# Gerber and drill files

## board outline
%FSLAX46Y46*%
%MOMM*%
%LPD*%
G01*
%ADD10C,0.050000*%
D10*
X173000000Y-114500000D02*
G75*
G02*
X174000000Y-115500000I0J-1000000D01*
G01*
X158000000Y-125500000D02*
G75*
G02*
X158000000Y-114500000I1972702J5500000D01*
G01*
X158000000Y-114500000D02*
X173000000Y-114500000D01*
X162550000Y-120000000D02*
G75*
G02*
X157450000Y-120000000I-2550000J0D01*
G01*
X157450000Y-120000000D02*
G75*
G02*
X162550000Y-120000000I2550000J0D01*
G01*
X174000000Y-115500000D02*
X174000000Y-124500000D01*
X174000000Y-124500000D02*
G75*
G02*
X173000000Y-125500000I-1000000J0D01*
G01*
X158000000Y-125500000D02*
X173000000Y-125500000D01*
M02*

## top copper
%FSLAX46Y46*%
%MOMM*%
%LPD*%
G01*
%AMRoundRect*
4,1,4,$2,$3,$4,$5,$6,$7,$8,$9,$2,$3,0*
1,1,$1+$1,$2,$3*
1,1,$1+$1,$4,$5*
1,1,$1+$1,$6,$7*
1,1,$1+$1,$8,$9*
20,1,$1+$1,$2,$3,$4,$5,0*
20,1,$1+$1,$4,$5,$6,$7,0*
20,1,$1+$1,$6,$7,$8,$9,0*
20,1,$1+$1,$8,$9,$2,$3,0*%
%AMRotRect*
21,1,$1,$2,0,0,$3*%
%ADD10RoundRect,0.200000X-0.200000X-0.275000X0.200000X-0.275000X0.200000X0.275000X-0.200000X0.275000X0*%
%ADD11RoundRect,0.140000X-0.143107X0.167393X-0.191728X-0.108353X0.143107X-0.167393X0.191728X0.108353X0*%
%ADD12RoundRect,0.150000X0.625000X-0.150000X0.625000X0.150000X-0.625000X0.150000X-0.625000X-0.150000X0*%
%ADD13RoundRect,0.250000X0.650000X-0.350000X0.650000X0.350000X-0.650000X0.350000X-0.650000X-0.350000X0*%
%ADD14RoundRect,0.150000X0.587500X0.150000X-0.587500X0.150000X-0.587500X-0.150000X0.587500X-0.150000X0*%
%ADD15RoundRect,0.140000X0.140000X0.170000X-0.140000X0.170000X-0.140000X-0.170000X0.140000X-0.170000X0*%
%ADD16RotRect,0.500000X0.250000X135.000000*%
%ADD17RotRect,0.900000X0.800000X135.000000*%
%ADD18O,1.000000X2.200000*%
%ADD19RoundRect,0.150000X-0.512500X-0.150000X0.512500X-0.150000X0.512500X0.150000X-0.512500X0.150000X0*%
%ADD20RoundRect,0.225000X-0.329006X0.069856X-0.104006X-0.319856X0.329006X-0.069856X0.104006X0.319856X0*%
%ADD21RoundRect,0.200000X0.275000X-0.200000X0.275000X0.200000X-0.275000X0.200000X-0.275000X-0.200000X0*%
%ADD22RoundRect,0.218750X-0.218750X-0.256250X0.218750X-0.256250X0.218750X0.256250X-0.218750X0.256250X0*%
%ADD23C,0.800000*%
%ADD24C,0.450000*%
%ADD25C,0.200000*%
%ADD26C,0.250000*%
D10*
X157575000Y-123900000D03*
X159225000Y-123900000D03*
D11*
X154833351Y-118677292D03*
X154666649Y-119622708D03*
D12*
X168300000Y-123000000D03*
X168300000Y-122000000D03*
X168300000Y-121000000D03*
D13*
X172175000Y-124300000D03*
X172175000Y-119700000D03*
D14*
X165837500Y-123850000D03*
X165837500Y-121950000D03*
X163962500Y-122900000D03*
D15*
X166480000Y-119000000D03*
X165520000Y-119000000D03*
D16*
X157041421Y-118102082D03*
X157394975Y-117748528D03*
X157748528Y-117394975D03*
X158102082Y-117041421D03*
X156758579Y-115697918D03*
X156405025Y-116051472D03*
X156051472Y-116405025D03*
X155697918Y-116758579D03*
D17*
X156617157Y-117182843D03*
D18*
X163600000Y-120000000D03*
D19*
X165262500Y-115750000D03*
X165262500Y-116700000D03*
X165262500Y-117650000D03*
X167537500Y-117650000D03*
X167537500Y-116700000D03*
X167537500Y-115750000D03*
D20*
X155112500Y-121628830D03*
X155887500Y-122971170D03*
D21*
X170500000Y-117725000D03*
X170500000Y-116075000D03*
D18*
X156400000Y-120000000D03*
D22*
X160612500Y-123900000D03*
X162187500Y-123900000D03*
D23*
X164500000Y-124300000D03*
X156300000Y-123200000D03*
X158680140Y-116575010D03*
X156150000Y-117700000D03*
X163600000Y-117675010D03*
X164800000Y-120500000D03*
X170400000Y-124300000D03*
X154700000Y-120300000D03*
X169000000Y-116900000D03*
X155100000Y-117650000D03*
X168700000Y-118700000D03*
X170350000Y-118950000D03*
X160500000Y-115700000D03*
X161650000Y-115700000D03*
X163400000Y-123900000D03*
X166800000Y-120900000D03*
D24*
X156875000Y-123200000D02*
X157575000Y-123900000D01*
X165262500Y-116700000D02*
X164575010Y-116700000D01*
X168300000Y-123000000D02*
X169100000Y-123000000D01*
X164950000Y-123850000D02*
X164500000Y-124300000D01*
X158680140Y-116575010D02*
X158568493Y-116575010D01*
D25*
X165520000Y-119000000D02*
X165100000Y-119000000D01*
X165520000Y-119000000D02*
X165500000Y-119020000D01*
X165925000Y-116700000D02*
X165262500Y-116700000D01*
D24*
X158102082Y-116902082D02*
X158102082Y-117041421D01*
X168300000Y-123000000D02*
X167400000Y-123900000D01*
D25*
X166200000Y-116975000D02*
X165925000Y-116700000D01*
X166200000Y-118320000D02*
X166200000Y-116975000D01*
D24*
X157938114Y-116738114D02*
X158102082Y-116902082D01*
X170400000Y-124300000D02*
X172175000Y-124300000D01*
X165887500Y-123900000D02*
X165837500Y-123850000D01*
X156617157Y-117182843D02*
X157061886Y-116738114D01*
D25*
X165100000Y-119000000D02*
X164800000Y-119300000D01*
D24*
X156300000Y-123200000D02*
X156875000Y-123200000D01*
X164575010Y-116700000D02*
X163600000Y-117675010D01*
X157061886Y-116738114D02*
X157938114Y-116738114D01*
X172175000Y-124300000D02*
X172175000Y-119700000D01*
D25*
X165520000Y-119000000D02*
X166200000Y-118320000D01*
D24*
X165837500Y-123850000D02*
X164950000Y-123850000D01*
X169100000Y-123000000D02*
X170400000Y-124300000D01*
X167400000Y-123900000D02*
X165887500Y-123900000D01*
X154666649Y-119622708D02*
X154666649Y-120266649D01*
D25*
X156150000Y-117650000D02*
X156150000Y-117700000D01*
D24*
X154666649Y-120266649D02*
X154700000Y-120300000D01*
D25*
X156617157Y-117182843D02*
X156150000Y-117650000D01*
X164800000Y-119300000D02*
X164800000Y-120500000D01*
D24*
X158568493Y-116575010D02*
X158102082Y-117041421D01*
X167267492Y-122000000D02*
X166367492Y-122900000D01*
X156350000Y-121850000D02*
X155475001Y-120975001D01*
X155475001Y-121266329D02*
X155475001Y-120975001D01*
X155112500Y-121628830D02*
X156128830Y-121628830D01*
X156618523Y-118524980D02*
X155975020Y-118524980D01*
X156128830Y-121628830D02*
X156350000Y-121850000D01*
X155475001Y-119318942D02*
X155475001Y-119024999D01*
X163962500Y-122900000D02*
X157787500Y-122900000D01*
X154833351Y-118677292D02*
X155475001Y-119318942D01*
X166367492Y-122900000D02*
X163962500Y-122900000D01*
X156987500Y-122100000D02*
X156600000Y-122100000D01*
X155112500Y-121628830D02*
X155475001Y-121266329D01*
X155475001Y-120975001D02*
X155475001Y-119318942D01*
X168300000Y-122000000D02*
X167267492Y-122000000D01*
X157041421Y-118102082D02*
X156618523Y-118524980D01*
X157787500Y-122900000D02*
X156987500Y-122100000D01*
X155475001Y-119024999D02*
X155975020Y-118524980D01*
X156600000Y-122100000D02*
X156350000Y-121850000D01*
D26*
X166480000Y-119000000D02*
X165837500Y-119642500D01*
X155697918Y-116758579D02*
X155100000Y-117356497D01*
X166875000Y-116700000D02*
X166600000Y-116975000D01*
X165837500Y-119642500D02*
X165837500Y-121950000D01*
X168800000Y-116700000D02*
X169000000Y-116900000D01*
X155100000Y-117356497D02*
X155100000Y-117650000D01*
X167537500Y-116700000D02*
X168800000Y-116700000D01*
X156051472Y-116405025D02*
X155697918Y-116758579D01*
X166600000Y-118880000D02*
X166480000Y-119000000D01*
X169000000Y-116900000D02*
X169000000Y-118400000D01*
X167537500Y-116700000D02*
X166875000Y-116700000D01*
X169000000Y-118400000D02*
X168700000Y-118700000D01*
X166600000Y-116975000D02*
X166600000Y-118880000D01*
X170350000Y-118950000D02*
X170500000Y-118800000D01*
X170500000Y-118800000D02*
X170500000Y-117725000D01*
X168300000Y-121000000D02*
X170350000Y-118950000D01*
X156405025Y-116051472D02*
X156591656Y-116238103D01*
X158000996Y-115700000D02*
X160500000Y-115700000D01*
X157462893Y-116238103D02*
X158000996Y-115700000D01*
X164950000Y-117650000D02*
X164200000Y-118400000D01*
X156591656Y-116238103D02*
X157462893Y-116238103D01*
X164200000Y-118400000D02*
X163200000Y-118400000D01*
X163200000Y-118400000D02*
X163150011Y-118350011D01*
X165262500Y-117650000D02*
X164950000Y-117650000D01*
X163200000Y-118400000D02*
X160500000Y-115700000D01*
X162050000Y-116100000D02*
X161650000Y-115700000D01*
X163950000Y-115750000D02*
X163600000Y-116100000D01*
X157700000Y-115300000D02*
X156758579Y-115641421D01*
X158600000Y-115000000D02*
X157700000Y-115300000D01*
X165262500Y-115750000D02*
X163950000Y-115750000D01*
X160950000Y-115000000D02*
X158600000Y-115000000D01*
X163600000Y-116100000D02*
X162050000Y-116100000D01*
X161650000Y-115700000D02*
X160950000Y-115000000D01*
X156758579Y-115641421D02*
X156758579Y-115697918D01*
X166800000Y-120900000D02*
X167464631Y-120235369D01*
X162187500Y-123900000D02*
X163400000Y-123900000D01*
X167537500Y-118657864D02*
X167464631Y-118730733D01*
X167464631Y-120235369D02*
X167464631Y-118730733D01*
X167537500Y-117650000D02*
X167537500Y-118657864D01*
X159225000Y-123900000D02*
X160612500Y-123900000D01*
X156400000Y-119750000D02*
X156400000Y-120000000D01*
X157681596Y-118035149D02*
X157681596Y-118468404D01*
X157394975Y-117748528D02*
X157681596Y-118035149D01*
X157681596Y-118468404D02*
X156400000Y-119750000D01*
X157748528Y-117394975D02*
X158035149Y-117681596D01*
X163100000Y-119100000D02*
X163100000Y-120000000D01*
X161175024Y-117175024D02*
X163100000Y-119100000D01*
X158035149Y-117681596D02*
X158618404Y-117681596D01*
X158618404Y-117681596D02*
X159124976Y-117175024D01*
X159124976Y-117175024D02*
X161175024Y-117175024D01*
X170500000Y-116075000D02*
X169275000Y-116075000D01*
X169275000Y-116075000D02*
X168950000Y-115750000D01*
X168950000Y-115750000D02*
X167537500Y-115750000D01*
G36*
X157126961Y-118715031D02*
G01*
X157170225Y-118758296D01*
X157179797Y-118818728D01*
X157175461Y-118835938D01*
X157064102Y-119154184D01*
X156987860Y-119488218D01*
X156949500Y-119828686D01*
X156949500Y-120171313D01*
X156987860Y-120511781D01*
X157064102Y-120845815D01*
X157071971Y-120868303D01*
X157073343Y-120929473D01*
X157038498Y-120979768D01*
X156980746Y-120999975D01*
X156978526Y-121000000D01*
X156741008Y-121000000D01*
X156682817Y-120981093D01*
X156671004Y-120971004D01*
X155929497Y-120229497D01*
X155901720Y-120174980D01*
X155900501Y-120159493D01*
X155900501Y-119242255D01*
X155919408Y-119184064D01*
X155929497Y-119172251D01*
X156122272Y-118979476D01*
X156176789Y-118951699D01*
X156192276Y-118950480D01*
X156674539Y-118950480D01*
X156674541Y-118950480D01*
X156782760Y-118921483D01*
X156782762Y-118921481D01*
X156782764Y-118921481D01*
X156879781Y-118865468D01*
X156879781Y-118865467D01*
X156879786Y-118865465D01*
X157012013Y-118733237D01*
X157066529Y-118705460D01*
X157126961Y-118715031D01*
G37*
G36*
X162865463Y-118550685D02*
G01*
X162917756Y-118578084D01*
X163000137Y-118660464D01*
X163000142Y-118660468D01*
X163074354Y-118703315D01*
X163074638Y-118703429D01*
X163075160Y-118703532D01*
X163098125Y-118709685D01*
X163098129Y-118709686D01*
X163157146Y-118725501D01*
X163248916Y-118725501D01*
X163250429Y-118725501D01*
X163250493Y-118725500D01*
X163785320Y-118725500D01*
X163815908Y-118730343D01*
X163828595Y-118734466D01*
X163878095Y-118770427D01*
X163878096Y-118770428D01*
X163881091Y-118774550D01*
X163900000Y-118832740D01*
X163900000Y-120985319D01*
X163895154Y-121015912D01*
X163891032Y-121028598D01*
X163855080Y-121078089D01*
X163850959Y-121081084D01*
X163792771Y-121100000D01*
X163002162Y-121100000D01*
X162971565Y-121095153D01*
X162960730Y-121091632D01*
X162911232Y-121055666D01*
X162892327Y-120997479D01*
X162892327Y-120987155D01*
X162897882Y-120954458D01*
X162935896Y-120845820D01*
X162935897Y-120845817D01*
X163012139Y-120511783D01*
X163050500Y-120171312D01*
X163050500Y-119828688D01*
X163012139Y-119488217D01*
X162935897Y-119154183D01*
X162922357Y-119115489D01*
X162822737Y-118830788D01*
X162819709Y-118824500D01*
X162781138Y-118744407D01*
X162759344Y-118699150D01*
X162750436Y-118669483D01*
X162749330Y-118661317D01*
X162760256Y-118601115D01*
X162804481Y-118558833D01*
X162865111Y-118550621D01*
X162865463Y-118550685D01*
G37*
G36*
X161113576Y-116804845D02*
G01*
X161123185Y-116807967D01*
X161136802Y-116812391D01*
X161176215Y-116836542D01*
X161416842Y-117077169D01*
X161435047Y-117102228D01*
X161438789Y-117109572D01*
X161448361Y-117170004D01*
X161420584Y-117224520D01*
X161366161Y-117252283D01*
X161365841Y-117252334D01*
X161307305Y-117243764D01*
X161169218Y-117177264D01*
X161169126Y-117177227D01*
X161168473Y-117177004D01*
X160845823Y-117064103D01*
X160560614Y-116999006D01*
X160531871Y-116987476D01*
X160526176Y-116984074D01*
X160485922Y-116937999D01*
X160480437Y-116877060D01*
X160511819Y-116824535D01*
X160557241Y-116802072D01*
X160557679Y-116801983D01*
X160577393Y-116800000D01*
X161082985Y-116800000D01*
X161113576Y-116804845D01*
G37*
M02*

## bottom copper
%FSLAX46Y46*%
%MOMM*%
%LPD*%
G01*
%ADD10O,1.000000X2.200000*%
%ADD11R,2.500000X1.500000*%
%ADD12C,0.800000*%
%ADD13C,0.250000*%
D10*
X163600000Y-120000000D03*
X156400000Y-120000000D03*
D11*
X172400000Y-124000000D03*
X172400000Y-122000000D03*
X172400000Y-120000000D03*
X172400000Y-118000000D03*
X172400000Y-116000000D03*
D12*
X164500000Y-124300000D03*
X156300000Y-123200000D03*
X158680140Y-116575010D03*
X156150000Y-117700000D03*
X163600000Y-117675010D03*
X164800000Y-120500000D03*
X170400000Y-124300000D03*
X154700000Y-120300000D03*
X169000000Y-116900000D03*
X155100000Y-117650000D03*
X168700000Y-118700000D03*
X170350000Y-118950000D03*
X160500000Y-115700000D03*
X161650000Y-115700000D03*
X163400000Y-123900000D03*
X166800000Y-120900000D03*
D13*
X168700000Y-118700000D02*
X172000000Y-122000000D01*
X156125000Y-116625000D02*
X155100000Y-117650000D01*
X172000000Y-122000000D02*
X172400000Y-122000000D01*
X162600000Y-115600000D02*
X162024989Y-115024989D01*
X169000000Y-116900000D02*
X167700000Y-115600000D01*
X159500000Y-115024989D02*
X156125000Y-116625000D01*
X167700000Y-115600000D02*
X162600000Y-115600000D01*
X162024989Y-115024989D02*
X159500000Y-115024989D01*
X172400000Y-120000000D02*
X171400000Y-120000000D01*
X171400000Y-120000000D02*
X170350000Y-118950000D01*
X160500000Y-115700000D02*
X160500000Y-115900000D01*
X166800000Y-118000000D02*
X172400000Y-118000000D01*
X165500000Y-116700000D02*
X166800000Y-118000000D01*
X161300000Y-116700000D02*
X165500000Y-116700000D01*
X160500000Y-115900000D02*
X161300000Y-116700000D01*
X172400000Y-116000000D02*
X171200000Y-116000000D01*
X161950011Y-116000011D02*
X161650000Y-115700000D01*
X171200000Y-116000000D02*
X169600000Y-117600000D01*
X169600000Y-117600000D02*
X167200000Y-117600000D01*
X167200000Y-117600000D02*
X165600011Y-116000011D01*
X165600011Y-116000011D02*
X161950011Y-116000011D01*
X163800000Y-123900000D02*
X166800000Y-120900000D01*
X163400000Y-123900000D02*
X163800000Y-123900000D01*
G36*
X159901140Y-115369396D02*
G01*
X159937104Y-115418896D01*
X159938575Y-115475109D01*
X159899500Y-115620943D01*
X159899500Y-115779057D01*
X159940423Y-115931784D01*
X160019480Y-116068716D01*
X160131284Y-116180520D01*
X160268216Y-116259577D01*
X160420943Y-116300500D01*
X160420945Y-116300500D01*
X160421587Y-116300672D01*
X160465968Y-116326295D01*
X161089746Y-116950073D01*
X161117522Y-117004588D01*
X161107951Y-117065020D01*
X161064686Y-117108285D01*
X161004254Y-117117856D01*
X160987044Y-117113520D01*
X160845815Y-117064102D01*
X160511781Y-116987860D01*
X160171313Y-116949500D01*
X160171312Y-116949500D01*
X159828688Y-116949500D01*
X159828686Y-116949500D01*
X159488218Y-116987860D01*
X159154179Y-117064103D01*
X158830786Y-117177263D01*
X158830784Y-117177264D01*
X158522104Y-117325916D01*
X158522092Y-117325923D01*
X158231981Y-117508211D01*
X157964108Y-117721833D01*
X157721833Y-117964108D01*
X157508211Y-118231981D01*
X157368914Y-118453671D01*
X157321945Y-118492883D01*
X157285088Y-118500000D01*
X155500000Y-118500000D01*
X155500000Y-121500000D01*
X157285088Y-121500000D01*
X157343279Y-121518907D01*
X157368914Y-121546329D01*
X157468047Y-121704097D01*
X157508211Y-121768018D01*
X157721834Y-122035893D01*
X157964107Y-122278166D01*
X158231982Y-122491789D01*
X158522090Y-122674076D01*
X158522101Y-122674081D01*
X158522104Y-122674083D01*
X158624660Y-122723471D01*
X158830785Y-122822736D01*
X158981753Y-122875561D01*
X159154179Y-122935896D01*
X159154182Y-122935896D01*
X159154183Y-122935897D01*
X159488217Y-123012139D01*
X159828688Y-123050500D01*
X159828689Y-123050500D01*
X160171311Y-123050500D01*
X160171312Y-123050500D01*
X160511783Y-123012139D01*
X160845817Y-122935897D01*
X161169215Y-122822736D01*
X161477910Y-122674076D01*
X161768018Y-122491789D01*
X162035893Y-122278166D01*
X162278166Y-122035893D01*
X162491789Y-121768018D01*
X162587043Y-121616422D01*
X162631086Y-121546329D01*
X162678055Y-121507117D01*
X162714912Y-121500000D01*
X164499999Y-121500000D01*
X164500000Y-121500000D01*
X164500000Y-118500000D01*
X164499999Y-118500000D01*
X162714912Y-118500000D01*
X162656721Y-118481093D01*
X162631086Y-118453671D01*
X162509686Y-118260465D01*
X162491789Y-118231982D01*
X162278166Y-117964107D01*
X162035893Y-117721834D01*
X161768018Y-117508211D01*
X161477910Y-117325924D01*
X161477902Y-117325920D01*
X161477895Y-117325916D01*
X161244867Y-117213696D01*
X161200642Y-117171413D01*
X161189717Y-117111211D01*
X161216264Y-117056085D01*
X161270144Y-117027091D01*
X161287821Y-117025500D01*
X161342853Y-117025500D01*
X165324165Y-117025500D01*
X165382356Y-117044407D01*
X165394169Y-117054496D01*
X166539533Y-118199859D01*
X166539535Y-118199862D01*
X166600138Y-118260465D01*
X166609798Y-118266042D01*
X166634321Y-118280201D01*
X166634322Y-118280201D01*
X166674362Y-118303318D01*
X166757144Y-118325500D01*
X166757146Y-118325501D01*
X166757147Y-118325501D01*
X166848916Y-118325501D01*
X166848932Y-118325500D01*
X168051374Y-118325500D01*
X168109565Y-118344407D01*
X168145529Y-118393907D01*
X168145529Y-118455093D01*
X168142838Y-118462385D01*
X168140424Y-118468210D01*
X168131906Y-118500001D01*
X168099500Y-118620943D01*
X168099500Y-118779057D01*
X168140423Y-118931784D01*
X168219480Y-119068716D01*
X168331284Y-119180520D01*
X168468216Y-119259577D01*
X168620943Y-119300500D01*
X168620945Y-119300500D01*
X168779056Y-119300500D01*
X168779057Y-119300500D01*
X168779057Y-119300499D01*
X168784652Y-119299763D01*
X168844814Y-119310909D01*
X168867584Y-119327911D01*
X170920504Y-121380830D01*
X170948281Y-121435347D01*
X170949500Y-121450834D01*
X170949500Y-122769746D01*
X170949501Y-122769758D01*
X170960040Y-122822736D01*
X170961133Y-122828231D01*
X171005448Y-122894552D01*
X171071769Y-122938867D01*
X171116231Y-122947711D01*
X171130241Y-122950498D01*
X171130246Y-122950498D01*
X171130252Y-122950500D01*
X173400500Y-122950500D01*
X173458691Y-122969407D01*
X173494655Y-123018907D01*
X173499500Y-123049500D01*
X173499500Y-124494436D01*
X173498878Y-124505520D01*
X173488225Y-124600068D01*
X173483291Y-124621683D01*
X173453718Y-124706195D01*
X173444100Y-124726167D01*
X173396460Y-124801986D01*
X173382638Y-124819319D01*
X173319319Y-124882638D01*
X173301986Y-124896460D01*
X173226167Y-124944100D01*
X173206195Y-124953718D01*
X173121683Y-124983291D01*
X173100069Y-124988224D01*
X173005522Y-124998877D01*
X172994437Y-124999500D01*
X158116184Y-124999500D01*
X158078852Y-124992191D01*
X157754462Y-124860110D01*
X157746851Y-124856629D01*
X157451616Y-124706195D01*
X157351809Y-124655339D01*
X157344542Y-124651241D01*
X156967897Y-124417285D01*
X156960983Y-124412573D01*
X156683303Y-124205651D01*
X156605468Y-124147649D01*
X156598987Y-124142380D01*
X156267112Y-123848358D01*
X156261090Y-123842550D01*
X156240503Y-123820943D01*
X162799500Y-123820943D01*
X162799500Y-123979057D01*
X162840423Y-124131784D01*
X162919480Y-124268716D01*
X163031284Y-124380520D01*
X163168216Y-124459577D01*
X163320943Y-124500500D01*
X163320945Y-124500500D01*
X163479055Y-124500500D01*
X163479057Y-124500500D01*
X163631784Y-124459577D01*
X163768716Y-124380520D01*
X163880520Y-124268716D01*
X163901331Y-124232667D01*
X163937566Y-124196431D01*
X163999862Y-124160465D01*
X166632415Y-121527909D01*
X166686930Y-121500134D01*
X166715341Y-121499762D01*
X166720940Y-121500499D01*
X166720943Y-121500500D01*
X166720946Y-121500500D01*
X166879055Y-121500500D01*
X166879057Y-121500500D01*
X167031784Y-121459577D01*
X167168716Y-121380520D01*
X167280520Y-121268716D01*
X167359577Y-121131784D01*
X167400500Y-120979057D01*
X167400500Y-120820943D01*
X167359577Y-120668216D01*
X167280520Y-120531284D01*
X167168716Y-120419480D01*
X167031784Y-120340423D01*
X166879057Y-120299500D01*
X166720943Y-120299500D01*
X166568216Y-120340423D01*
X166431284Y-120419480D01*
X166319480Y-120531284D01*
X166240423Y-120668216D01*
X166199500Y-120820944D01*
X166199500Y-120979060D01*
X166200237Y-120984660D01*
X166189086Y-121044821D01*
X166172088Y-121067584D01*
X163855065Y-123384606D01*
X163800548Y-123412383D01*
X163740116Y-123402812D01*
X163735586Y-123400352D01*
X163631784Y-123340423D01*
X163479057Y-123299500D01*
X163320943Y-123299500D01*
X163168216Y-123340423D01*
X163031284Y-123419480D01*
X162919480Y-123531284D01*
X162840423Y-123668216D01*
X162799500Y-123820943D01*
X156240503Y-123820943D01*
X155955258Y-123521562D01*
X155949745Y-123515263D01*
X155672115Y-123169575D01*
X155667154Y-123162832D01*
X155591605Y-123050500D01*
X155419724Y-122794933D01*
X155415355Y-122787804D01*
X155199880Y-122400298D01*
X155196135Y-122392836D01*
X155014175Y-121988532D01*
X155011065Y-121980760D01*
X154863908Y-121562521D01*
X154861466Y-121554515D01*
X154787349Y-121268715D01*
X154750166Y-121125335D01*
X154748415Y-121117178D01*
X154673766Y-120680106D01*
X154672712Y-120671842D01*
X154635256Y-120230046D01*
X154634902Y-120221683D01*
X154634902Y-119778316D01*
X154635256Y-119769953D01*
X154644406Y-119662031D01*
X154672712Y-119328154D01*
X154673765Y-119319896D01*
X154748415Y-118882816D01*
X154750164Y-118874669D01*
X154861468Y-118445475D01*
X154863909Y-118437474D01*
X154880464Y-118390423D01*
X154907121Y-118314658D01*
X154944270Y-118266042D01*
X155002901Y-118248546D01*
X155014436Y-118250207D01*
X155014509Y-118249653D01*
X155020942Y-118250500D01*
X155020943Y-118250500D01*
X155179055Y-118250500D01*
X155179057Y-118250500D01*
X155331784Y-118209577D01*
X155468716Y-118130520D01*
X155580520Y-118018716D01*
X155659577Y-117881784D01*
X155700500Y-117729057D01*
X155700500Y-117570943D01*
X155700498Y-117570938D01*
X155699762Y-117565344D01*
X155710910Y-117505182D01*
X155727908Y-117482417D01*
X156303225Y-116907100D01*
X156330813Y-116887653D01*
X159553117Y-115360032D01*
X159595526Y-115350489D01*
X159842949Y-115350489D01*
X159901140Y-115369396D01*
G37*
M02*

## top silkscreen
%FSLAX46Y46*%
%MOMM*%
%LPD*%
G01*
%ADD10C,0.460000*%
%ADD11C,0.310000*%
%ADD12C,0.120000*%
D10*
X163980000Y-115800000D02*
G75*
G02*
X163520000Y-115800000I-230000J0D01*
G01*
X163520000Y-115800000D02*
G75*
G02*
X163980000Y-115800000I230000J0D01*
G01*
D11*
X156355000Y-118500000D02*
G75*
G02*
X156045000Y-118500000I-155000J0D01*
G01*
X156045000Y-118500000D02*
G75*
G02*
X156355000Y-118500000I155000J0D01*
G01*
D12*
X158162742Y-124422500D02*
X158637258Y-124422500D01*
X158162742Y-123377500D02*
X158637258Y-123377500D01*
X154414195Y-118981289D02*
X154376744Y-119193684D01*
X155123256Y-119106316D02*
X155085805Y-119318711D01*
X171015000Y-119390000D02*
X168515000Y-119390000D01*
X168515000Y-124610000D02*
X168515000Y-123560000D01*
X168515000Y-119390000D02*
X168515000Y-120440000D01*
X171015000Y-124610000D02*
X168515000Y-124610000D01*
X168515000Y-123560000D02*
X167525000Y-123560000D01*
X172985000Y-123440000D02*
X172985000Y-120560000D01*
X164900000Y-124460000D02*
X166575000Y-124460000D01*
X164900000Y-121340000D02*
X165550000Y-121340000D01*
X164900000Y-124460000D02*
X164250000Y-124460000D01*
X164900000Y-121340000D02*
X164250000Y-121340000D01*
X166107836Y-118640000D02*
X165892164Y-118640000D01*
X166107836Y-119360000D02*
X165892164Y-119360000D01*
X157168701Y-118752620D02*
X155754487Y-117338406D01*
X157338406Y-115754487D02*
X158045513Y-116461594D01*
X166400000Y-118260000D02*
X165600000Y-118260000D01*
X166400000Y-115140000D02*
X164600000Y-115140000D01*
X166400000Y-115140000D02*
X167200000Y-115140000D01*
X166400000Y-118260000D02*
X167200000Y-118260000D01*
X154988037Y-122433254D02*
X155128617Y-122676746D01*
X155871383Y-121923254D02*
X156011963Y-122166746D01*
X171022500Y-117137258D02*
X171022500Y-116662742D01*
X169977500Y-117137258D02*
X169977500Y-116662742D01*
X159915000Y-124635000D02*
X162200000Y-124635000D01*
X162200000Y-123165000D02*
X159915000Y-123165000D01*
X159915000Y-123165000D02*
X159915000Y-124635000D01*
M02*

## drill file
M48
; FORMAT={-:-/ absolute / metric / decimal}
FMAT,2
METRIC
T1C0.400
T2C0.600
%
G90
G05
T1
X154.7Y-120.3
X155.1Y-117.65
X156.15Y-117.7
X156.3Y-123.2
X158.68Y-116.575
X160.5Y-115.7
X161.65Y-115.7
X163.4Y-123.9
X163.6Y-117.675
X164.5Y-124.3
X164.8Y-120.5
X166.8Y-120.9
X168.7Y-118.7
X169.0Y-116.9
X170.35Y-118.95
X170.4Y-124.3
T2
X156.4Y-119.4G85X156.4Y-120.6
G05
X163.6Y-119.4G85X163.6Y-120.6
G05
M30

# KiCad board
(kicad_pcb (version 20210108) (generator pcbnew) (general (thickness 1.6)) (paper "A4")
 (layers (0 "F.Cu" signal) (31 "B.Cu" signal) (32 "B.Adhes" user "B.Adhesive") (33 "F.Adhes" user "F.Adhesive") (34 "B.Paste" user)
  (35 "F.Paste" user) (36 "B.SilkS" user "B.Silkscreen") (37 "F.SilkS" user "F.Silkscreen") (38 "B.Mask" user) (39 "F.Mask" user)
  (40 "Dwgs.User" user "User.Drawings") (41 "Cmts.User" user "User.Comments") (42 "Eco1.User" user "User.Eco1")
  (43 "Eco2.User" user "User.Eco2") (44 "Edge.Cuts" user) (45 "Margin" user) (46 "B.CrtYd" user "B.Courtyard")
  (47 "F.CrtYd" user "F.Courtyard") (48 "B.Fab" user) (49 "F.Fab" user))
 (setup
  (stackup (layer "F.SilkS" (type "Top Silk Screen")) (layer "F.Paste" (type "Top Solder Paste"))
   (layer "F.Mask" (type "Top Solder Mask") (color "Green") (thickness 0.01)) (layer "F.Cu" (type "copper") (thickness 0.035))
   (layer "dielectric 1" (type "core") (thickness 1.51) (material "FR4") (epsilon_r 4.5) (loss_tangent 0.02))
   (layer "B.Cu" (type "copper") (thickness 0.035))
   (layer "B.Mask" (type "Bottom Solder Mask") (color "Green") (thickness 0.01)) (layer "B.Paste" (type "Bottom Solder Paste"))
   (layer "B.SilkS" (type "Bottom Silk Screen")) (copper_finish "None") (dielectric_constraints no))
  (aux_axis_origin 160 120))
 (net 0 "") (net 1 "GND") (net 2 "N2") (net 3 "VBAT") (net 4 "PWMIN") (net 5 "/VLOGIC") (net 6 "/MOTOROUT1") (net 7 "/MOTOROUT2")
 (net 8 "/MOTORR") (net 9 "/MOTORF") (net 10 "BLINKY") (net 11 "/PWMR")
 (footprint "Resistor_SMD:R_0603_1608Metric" (layer "F.Cu") (at 158.4 123.9)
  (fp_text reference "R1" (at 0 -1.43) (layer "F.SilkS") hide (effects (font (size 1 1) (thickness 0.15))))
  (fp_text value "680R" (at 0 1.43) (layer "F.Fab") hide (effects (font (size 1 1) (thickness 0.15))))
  (fp_line (start -0.237258 0.5225) (end 0.237258 0.5225) (layer "F.SilkS") (width 0.12))
  (fp_line (start -0.237258 -0.5225) (end 0.237258 -0.5225) (layer "F.SilkS") (width 0.12))
  (pad "1" smd roundrect (at -0.825 0) (locked) (size 0.8 0.95) (layers "F.Cu" "F.Paste" "F.Mask") (roundrect_rratio 0.25) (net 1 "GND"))
  (pad "2" smd roundrect (at 0.825 0) (locked) (size 0.8 0.95) (layers "F.Cu" "F.Paste" "F.Mask") (roundrect_rratio 0.25) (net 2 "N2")))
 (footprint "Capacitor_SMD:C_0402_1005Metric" (layer "F.Cu") (at 154.75 119.15 -100)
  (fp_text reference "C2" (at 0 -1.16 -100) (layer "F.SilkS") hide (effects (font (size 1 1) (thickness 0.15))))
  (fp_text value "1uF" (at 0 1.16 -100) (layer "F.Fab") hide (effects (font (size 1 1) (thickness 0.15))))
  (fp_line (start -0.107836 0.36) (end 0.107836 0.36) (layer "F.SilkS") (width 0.12))
  (fp_line (start -0.107836 -0.36) (end 0.107836 -0.36) (layer "F.SilkS") (width 0.12))
  (pad "1" smd roundrect (at -0.48 0 260) (locked) (size 0.56 0.62) (layers "F.Cu" "F.Paste" "F.Mask") (roundrect_rratio 0.25)
   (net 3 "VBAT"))
  (pad "2" smd roundrect (at 0.48 0 260) (locked) (size 0.56 0.62) (layers "F.Cu" "F.Paste" "F.Mask") (roundrect_rratio 0.25) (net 1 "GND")))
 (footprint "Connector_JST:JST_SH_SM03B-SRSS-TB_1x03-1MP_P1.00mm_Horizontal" (layer "F.Cu") (at 170.3 122 90)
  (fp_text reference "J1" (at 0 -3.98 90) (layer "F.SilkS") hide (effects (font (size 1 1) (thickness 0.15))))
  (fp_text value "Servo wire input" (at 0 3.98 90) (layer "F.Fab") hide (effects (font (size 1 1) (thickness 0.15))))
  (fp_line (start 2.61 0.715) (end 2.61 -1.785) (layer "F.SilkS") (width 0.12))
  (fp_line (start -2.61 -1.785) (end -1.56 -1.785) (layer "F.SilkS") (width 0.12))
  (fp_line (start 2.61 -1.785) (end 1.56 -1.785) (layer "F.SilkS") (width 0.12))
  (fp_line (start -2.61 0.715) (end -2.61 -1.785) (layer "F.SilkS") (width 0.12))
  (fp_line (start -1.56 -1.785) (end -1.56 -2.775) (layer "F.SilkS") (width 0.12))
  (fp_line (start -1.44 2.685) (end 1.44 2.685) (layer "F.SilkS") (width 0.12))
  (pad "1" smd roundrect (at -1 -2 90) (locked) (size 0.6 1.55) (layers "F.Cu" "F.Paste" "F.Mask") (roundrect_rratio 0.25) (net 1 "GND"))
  (pad "2" smd roundrect (at 0 -2 90) (locked) (size 0.6 1.55) (layers "F.Cu" "F.Paste" "F.Mask") (roundrect_rratio 0.25) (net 3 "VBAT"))
  (pad "3" smd roundrect (at 1 -2 90) (locked) (size 0.6 1.55) (layers "F.Cu" "F.Paste" "F.Mask") (roundrect_rratio 0.25) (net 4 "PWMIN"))
  (pad "MP" smd roundrect (at -2.3 1.875 90) (locked) (size 1.2 1.8) (layers "F.Cu" "F.Paste" "F.Mask") (roundrect_rratio 0.208333)
   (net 1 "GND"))
  (pad "MP" smd roundrect (at 2.3 1.875 90) (locked) (size 1.2 1.8) (layers "F.Cu" "F.Paste" "F.Mask") (roundrect_rratio 0.208333)
   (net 1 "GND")))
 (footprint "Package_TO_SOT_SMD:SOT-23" (layer "F.Cu") (at 164.9 122.9 180)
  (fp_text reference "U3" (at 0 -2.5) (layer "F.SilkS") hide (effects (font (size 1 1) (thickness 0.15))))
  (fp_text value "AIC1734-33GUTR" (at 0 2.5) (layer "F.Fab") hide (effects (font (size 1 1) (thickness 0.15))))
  (fp_line (start 0 -1.56) (end -1.675 -1.56) (layer "F.SilkS") (width 0.12))
  (fp_line (start 0 1.56) (end -0.65 1.56) (layer "F.SilkS") (width 0.12))
  (fp_line (start 0 -1.56) (end 0.65 -1.56) (layer "F.SilkS") (width 0.12))
  (fp_line (start 0 1.56) (end 0.65 1.56) (layer "F.SilkS") (width 0.12))
  (pad "1" smd roundrect (at -0.9375 -0.95 180) (locked) (size 1.475 0.6) (layers "F.Cu" "F.Paste" "F.Mask") (roundrect_rratio 0.25)
   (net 1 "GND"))
  (pad "2" smd roundrect (at -0.9375 0.95 180) (locked) (size 1.475 0.6) (layers "F.Cu" "F.Paste" "F.Mask") (roundrect_rratio 0.25)
   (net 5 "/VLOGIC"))
  (pad "3" smd roundrect (at 0.9375 0 180) (locked) (size 1.475 0.6) (layers "F.Cu" "F.Paste" "F.Mask") (roundrect_rratio 0.25)
   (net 3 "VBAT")))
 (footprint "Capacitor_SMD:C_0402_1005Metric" (layer "F.Cu") (at 166 119 180)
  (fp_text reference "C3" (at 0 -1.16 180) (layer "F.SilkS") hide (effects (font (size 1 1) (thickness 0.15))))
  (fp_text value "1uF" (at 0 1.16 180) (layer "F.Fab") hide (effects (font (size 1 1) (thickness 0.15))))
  (fp_line (start -0.107836 0.36) (end 0.107836 0.36) (layer "F.SilkS") (width 0.12))
  (fp_line (start -0.107836 -0.36) (end 0.107836 -0.36) (layer "F.SilkS") (width 0.12))
  (pad "1" smd roundrect (at -0.48 0 180) (locked) (size 0.56 0.62) (layers "F.Cu" "F.Paste" "F.Mask") (roundrect_rratio 0.25)
   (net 5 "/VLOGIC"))
  (pad "2" smd roundrect (at 0.48 0 180) (locked) (size 0.56 0.62) (layers "F.Cu" "F.Paste" "F.Mask") (roundrect_rratio 0.25) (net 1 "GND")))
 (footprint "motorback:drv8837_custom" (layer "F.Cu") (at 156.9 116.9 135)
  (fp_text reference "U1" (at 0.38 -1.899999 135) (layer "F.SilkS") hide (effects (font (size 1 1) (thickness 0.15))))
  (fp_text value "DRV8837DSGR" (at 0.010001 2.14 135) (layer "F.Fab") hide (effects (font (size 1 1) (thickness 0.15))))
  (fp_line (start -1.5 -1.12) (end 0.5 -1.12) (layer "F.SilkS") (width 0.12))
  (fp_line (start 0.5 1.12) (end -0.5 1.12) (layer "F.SilkS") (width 0.12))
  (pad "" smd rect (at 0 -0.4 135) (locked) (size 0.75 0.65) (layers "F.Paste"))
  (pad "1" smd rect (at -0.95 -0.75 135) (locked) (size 0.5 0.25) (layers "F.Cu" "F.Paste" "F.Mask") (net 3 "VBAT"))
  (pad "2" smd rect (at -0.95 -0.25 135) (locked) (size 0.5 0.25) (layers "F.Cu" "F.Paste" "F.Mask") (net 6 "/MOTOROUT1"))
  (pad "3" smd rect (at -0.95 0.25 135) (locked) (size 0.5 0.25) (layers "F.Cu" "F.Paste" "F.Mask") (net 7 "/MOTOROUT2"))
  (pad "4" smd rect (at -0.95 0.75 135) (locked) (size 0.5 0.25) (layers "F.Cu" "F.Paste" "F.Mask") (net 1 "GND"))
  (pad "5" smd rect (at 0.95 0.75 135) (locked) (size 0.5 0.25) (layers "F.Cu" "F.Paste" "F.Mask") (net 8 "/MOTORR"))
  (pad "6" smd rect (at 0.95 0.25 135) (locked) (size 0.5 0.25) (layers "F.Cu" "F.Paste" "F.Mask") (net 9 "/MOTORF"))
  (pad "7" smd rect (at 0.95 -0.25 135) (locked) (size 0.5 0.25) (layers "F.Cu" "F.Paste" "F.Mask") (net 5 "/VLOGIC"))
  (pad "8" smd rect (at 0.95 -0.75 135) (locked) (size 0.5 0.25) (layers "F.Cu" "F.Paste" "F.Mask") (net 5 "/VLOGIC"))
  (pad "9" smd rect (at 0 -0.4 135) (locked) (size 0.9 0.8) (layers "F.Cu" "F.Mask") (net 1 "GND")))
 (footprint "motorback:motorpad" (layer "F.Cu") (at 163.6 120)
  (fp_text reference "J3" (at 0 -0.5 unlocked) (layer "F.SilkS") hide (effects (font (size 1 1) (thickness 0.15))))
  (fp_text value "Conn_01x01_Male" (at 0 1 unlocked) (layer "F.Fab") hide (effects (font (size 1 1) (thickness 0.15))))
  (pad "1" thru_hole oval (at 0 0) (size 1 2.2) (drill oval 0.6 1.8) (layers *.Cu *.Mask) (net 7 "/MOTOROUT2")))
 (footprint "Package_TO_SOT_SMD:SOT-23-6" (layer "F.Cu") (at 166.4 116.7)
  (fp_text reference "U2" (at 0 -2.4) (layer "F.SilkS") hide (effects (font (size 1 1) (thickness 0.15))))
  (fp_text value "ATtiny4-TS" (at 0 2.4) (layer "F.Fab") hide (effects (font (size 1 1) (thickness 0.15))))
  (fp_line (start 0 1.56) (end -0.8 1.56) (layer "F.SilkS") (width 0.12))
  (fp_line (start 0 -1.56) (end -1.8 -1.56) (layer "F.SilkS") (width 0.12))
  (fp_line (start 0 -1.56) (end 0.8 -1.56) (layer "F.SilkS") (width 0.12))
  (fp_line (start 0 1.56) (end 0.8 1.56) (layer "F.SilkS") (width 0.12))
  (pad "1" smd roundrect (at -1.1375 -0.95) (locked) (size 1.325 0.6) (layers "F.Cu" "F.Paste" "F.Mask") (roundrect_rratio 0.25)
   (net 8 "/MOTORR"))
  (pad "2" smd roundrect (at -1.1375 0) (locked) (size 1.325 0.6) (layers "F.Cu" "F.Paste" "F.Mask") (roundrect_rratio 0.25) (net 1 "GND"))
  (pad "3" smd roundrect (at -1.1375 0.95) (locked) (size 1.325 0.6) (layers "F.Cu" "F.Paste" "F.Mask") (roundrect_rratio 0.25)
   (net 9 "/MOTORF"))
  (pad "4" smd roundrect (at 1.1375 0.95) (locked) (size 1.325 0.6) (layers "F.Cu" "F.Paste" "F.Mask") (roundrect_rratio 0.25)
   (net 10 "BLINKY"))
  (pad "5" smd roundrect (at 1.1375 0) (locked) (size 1.325 0.6) (layers "F.Cu" "F.Paste" "F.Mask") (roundrect_rratio 0.25)
   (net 5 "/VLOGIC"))
  (pad "6" smd roundrect (at 1.1375 -0.95) (locked) (size 1.325 0.6) (layers "F.Cu" "F.Paste" "F.Mask") (roundrect_rratio 0.25)
   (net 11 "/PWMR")))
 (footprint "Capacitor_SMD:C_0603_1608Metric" (layer "F.Cu") (at 155.5 122.3 -60)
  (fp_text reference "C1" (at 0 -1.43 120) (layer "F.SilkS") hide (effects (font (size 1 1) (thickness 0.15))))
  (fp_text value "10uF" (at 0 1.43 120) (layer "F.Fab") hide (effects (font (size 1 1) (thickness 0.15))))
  (fp_line (start -0.14058 0.51) (end 0.14058 0.51) (layer "F.SilkS") (width 0.12))
  (fp_line (start -0.14058 -0.51) (end 0.14058 -0.51) (layer "F.SilkS") (width 0.12))
  (pad "1" smd roundrect (at -0.775 0 300) (locked) (size 0.9 0.95) (layers "F.Cu" "F.Paste" "F.Mask") (roundrect_rratio 0.25)
   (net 3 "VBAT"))
  (pad "2" smd roundrect (at 0.775 0 300) (locked) (size 0.9 0.95) (layers "F.Cu" "F.Paste" "F.Mask") (roundrect_rratio 0.25) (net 1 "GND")))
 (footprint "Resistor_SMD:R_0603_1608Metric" (layer "F.Cu") (at 170.5 116.9 90)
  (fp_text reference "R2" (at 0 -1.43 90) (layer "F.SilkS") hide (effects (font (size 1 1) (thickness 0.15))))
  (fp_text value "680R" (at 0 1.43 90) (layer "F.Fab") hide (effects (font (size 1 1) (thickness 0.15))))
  (fp_line (start -0.237258 0.5225) (end 0.237258 0.5225) (layer "F.SilkS") (width 0.12))
  (fp_line (start -0.237258 -0.5225) (end 0.237258 -0.5225) (layer "F.SilkS") (width 0.12))
  (pad "1" smd roundrect (at -0.825 0 90) (locked) (size 0.8 0.95) (layers "F.Cu" "F.Paste" "F.Mask") (roundrect_rratio 0.25)
   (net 4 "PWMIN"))
  (pad "2" smd roundrect (at 0.825 0 90) (locked) (size 0.8 0.95) (layers "F.Cu" "F.Paste" "F.Mask") (roundrect_rratio 0.25)
   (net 11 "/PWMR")))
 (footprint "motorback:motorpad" (layer "F.Cu") (at 156.4 120)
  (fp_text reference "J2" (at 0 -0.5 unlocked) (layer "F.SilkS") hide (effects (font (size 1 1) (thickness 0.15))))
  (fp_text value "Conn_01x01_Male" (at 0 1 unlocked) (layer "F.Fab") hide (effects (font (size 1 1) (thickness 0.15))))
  (pad "1" thru_hole oval (at 0 0) (size 1 2.2) (drill oval 0.6 1.8) (layers *.Cu *.Mask) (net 6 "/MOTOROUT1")))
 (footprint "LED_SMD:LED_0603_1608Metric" (layer "F.Cu") (at 161.4 123.9)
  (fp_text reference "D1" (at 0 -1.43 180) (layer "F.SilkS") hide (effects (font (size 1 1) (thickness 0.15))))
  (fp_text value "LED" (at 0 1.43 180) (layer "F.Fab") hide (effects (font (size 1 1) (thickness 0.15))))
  (fp_line (start -1.485 0.735) (end 0.8 0.735) (layer "F.SilkS") (width 0.12))
  (fp_line (start 0.8 -0.735) (end -1.485 -0.735) (layer "F.SilkS") (width 0.12))
  (fp_line (start -1.485 -0.735) (end -1.485 0.735) (layer "F.SilkS") (width 0.12))
  (pad "1" smd roundrect (at -0.7875 0) (locked) (size 0.875 0.95) (layers "F.Cu" "F.Paste" "F.Mask") (roundrect_rratio 0.25) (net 2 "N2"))
  (pad "2" smd roundrect (at 0.7875 0) (locked) (size 0.875 0.95) (layers "F.Cu" "F.Paste" "F.Mask") (roundrect_rratio 0.25)
   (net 10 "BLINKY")))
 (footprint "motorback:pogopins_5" (layer "B.Cu") (at 172.4 120 90)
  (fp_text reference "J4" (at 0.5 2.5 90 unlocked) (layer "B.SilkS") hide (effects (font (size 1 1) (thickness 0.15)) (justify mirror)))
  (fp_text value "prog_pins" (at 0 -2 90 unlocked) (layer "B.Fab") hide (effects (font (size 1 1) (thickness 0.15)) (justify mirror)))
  (pad "1" smd rect (at -4 0 90) (size 1.5 2.5) (layers "B.Cu" "B.Paste" "B.Mask") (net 1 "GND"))
  (pad "2" smd rect (at -2 0 90) (size 1.5 2.5) (layers "B.Cu" "B.Paste" "B.Mask") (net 5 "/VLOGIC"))
  (pad "3" smd rect (at 0 0 90) (size 1.5 2.5) (layers "B.Cu" "B.Paste" "B.Mask") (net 4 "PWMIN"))
  (pad "4" smd rect (at 2 0 90) (size 1.5 2.5) (layers "B.Cu" "B.Paste" "B.Mask") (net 9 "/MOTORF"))
  (pad "5" smd rect (at 4 0 90) (size 1.5 2.5) (layers "B.Cu" "B.Paste" "B.Mask") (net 8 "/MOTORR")))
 (gr_circle (center 163.75 115.8) (end 164.15 115.8) (layer "F.SilkS") (width 0.12) (fill solid))
 (gr_circle (center 156.2 118.5) (end 156.45 118.5) (layer "F.SilkS") (width 0.12) (fill solid))
 (gr_arc (start 173 115.5) (end 174 115.5) (angle -90) (layer "Edge.Cuts") (width 0.05))
 (gr_arc (start 159.972702 120) (end 158 114.5) (angle -140.5369116) (layer "Edge.Cuts") (width 0.05))
 (gr_line (start 158 114.5) (end 173 114.5) (layer "Edge.Cuts") (width 0.05))
 (gr_circle (center 160 120) (end 162.55 120) (layer "Edge.Cuts") (width 0.05) (fill none))
 (gr_line (start 174 115.5) (end 174 124.5) (layer "Edge.Cuts") (width 0.05))
 (gr_arc (start 173 124.5) (end 173 125.5) (angle -90) (layer "Edge.Cuts") (width 0.05))
 (gr_line (start 158 125.5) (end 173 125.5) (layer "Edge.Cuts") (width 0.05))
 (segment (start 156.875 123.2) (end 157.575 123.9) (width 0.45) (layer "F.Cu") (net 1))
 (segment (start 165.2625 116.7) (end 164.57501 116.7) (width 0.45) (layer "F.Cu") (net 1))
 (segment (start 168.3 123) (end 169.1 123) (width 0.45) (layer "F.Cu") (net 1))
 (segment (start 164.95 123.85) (end 164.5 124.3) (width 0.45) (layer "F.Cu") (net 1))
 (segment (start 158.68014 116.57501) (end 158.568493 116.57501) (width 0.45) (layer "F.Cu") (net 1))
 (segment (start 165.52 119) (end 165.1 119) (width 0.2) (layer "F.Cu") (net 1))
 (segment (start 165.52 119) (end 165.5 119.02) (width 0.2) (layer "F.Cu") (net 1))
 (segment (start 165.925 116.7) (end 165.2625 116.7) (width 0.2) (layer "F.Cu") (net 1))
 (segment (start 158.102082 116.902082) (end 158.102082 117.041421) (width 0.45) (layer "F.Cu") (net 1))
 (segment (start 168.3 123) (end 167.4 123.9) (width 0.45) (layer "F.Cu") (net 1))
 (segment (start 166.2 116.975) (end 165.925 116.7) (width 0.2) (layer "F.Cu") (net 1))
 (segment (start 166.2 118.32) (end 166.2 116.975) (width 0.2) (layer "F.Cu") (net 1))
 (segment (start 157.938114 116.738114) (end 158.102082 116.902082) (width 0.45) (layer "F.Cu") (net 1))
 (segment (start 170.4 124.3) (end 172.175 124.3) (width 0.45) (layer "F.Cu") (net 1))
 (segment (start 165.8875 123.9) (end 165.8375 123.85) (width 0.45) (layer "F.Cu") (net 1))
 (segment (start 156.617157 117.182843) (end 157.061886 116.738114) (width 0.45) (layer "F.Cu") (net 1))
 (segment (start 165.1 119) (end 164.8 119.3) (width 0.2) (layer "F.Cu") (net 1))
 (segment (start 156.3 123.2) (end 156.875 123.2) (width 0.45) (layer "F.Cu") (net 1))
 (segment (start 164.57501 116.7) (end 163.6 117.67501) (width 0.45) (layer "F.Cu") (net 1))
 (segment (start 157.061886 116.738114) (end 157.938114 116.738114) (width 0.45) (layer "F.Cu") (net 1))
 (segment (start 172.175 124.3) (end 172.175 119.7) (width 0.45) (layer "F.Cu") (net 1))
 (segment (start 165.52 119) (end 166.2 118.32) (width 0.2) (layer "F.Cu") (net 1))
 (segment (start 165.8375 123.85) (end 164.95 123.85) (width 0.45) (layer "F.Cu") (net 1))
 (segment (start 169.1 123) (end 170.4 124.3) (width 0.45) (layer "F.Cu") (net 1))
 (segment (start 167.4 123.9) (end 165.8875 123.9) (width 0.45) (layer "F.Cu") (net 1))
 (segment (start 154.666649 119.622708) (end 154.666649 120.266649) (width 0.45) (layer "F.Cu") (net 1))
 (segment (start 156.15 117.65) (end 156.15 117.7) (width 0.2) (layer "F.Cu") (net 1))
 (segment (start 154.666649 120.266649) (end 154.7 120.3) (width 0.45) (layer "F.Cu") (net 1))
 (segment (start 156.617157 117.182843) (end 156.15 117.65) (width 0.2) (layer "F.Cu") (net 1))
 (segment (start 164.8 119.3) (end 164.8 120.5) (width 0.2) (layer "F.Cu") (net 1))
 (segment (start 158.568493 116.57501) (end 158.102082 117.041421) (width 0.45) (layer "F.Cu") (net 1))
 (via (at 164.5 124.3) (size 0.8) (drill 0.4) (layers "F.Cu" "B.Cu") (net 1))
 (via (at 156.3 123.2) (size 0.8) (drill 0.4) (layers "F.Cu" "B.Cu") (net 1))
 (via (at 158.68014 116.57501) (size 0.8) (drill 0.4) (layers "F.Cu" "B.Cu") (free) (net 1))
 (via (at 156.15 117.7) (size 0.8) (drill 0.4) (layers "F.Cu" "B.Cu") (free) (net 1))
 (via (at 163.6 117.67501) (size 0.8) (drill 0.4) (layers "F.Cu" "B.Cu") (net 1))
 (via (at 164.8 120.5) (size 0.8) (drill 0.4) (layers "F.Cu" "B.Cu") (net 1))
 (via (at 170.4 124.3) (size 0.8) (drill 0.4) (layers "F.Cu" "B.Cu") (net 1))
 (via (at 154.7 120.3) (size 0.8) (drill 0.4) (layers "F.Cu" "B.Cu") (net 1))
 (segment (start 167.267492 122) (end 166.367492 122.9) (width 0.45) (layer "F.Cu") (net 3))
 (segment (start 156.35 121.85) (end 155.475001 120.975001) (width 0.45) (layer "F.Cu") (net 3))
 (segment (start 155.475001 121.266329) (end 155.475001 120.975001) (width 0.45) (layer "F.Cu") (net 3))
 (segment (start 155.1125 121.62883) (end 156.12883 121.62883) (width 0.45) (layer "F.Cu") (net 3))
 (segment (start 156.618523 118.52498) (end 155.97502 118.52498) (width 0.45) (layer "F.Cu") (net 3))
 (segment (start 156.12883 121.62883) (end 156.35 121.85) (width 0.45) (layer "F.Cu") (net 3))
 (segment (start 155.475001 119.318942) (end 155.475001 119.024999) (width 0.45) (layer "F.Cu") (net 3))
 (segment (start 163.9625 122.9) (end 157.7875 122.9) (width 0.45) (layer "F.Cu") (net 3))
 (segment (start 154.833351 118.677292) (end 155.475001 119.318942) (width 0.45) (layer "F.Cu") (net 3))
 (segment (start 166.367492 122.9) (end 163.9625 122.9) (width 0.45) (layer "F.Cu") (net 3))
 (segment (start 156.9875 122.1) (end 156.6 122.1) (width 0.45) (layer "F.Cu") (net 3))
 (segment (start 155.1125 121.62883) (end 155.475001 121.266329) (width 0.45) (layer "F.Cu") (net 3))
 (segment (start 155.475001 120.975001) (end 155.475001 119.318942) (width 0.45) (layer "F.Cu") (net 3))
 (segment (start 168.3 122) (end 167.267492 122) (width 0.45) (layer "F.Cu") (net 3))
 (segment (start 157.041421 118.102082) (end 156.618523 118.52498) (width 0.45) (layer "F.Cu") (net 3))
 (segment (start 157.7875 122.9) (end 156.9875 122.1) (width 0.45) (layer "F.Cu") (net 3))
 (segment (start 155.475001 119.024999) (end 155.97502 118.52498) (width 0.45) (layer "F.Cu") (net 3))
 (segment (start 156.6 122.1) (end 156.35 121.85) (width 0.45) (layer "F.Cu") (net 3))
 (segment (start 166.48 119) (end 165.8375 119.6425) (width 0.25) (layer "F.Cu") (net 5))
 (segment (start 155.697918 116.758579) (end 155.1 117.356497) (width 0.25) (layer "F.Cu") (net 5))
 (segment (start 166.875 116.7) (end 166.6 116.975) (width 0.25) (layer "F.Cu") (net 5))
 (segment (start 165.8375 119.6425) (end 165.8375 121.95) (width 0.25) (layer "F.Cu") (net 5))
 (segment (start 168.8 116.7) (end 169 116.9) (width 0.25) (layer "F.Cu") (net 5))
 (segment (start 155.1 117.356497) (end 155.1 117.65) (width 0.25) (layer "F.Cu") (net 5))
 (segment (start 167.5375 116.7) (end 168.8 116.7) (width 0.25) (layer "F.Cu") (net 5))
 (segment (start 156.051472 116.405025) (end 155.697918 116.758579) (width 0.25) (layer "F.Cu") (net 5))
 (segment (start 166.6 118.88) (end 166.48 119) (width 0.25) (layer "F.Cu") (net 5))
 (segment (start 169 116.9) (end 169 118.4) (width 0.25) (layer "F.Cu") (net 5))
 (segment (start 167.5375 116.7) (end 166.875 116.7) (width 0.25) (layer "F.Cu") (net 5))
 (segment (start 169 118.4) (end 168.7 118.7) (width 0.25) (layer "F.Cu") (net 5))
 (segment (start 166.6 116.975) (end 166.6 118.88) (width 0.25) (layer "F.Cu") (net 5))
 (via (at 169 116.9) (size 0.8) (drill 0.4) (layers "F.Cu" "B.Cu") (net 5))
 (via (at 155.1 117.65) (size 0.8) (drill 0.4) (layers "F.Cu" "B.Cu") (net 5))
 (via (at 168.7 118.7) (size 0.8) (drill 0.4) (layers "F.Cu" "B.Cu") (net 5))
 (segment (start 168.7 118.7) (end 172 122) (width 0.25) (layer "B.Cu") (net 5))
 (segment (start 156.125 116.625) (end 155.1 117.65) (width 0.25) (layer "B.Cu") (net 5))
 (segment (start 172 122) (end 172.4 122) (width 0.25) (layer "B.Cu") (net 5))
 (segment (start 162.6 115.6) (end 162.024989 115.024989) (width 0.25) (layer "B.Cu") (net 5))
 (segment (start 169 116.9) (end 167.7 115.6) (width 0.25) (layer "B.Cu") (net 5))
 (segment (start 159.5 115.024989) (end 156.125 116.625) (width 0.25) (layer "B.Cu") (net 5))
 (segment (start 167.7 115.6) (end 162.6 115.6) (width 0.25) (layer "B.Cu") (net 5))
 (segment (start 162.024989 115.024989) (end 159.5 115.024989) (width 0.25) (layer "B.Cu") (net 5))
 (segment (start 170.35 118.95) (end 170.5 118.8) (width 0.25) (layer "F.Cu") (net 4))
 (segment (start 170.5 118.8) (end 170.5 117.725) (width 0.25) (layer "F.Cu") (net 4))
 (segment (start 168.3 121) (end 170.35 118.95) (width 0.25) (layer "F.Cu") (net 4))
 (via (at 170.35 118.95) (size 0.8) (drill 0.4) (layers "F.Cu" "B.Cu") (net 4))
 (segment (start 172.4 120) (end 171.4 120) (width 0.25) (layer "B.Cu") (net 4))
 (segment (start 171.4 120) (end 170.35 118.95) (width 0.25) (layer "B.Cu") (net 4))
 (segment (start 156.405025 116.051472) (end 156.591656 116.238103) (width 0.25) (layer "F.Cu") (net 9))
 (segment (start 158.000996 115.7) (end 160.5 115.7) (width 0.25) (layer "F.Cu") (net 9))
 (segment (start 157.462893 116.238103) (end 158.000996 115.7) (width 0.25) (layer "F.Cu") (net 9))
 (segment (start 164.95 117.65) (end 164.2 118.4) (width 0.25) (layer "F.Cu") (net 9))
 (segment (start 156.591656 116.238103) (end 157.462893 116.238103) (width 0.25) (layer "F.Cu") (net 9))
 (segment (start 164.2 118.4) (end 163.2 118.4) (width 0.25) (layer "F.Cu") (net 9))
 (segment (start 163.2 118.4) (end 163.150011 118.350011) (width 0.25) (layer "F.Cu") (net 9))
 (segment (start 165.2625 117.65) (end 164.95 117.65) (width 0.25) (layer "F.Cu") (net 9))
 (segment (start 163.2 118.4) (end 160.5 115.7) (width 0.25) (layer "F.Cu") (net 9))
 (via (at 160.5 115.7) (size 0.8) (drill 0.4) (layers "F.Cu" "B.Cu") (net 9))
 (segment (start 160.5 115.7) (end 160.5 115.9) (width 0.25) (layer "B.Cu") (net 9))
 (segment (start 166.8 118) (end 172.4 118) (width 0.25) (layer "B.Cu") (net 9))
 (segment (start 165.5 116.7) (end 166.8 118) (width 0.25) (layer "B.Cu") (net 9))
 (segment (start 161.3 116.7) (end 165.5 116.7) (width 0.25) (layer "B.Cu") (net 9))
 (segment (start 160.5 115.9) (end 161.3 116.7) (width 0.25) (layer "B.Cu") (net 9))
 (segment (start 162.05 116.1) (end 161.65 115.7) (width 0.25) (layer "F.Cu") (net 8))
 (segment (start 163.95 115.75) (end 163.6 116.1) (width 0.25) (layer "F.Cu") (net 8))
 (segment (start 157.7 115.3) (end 156.758579 115.641421) (width 0.25) (layer "F.Cu") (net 8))
 (segment (start 158.6 115) (end 157.7 115.3) (width 0.25) (layer "F.Cu") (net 8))
 (segment (start 165.2625 115.75) (end 163.95 115.75) (width 0.25) (layer "F.Cu") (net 8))
 (segment (start 160.95 115) (end 158.6 115) (width 0.25) (layer "F.Cu") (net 8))
 (segment (start 163.6 116.1) (end 162.05 116.1) (width 0.25) (layer "F.Cu") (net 8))
 (segment (start 161.65 115.7) (end 160.95 115) (width 0.25) (layer "F.Cu") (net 8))
 (segment (start 156.758579 115.641421) (end 156.758579 115.697918) (width 0.25) (layer "F.Cu") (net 8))
 (via (at 161.65 115.7) (size 0.8) (drill 0.4) (layers "F.Cu" "B.Cu") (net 8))
 (segment (start 172.4 116) (end 171.2 116) (width 0.25) (layer "B.Cu") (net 8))
 (segment (start 161.950011 116.000011) (end 161.65 115.7) (width 0.25) (layer "B.Cu") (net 8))
 (segment (start 171.2 116) (end 169.6 117.6) (width 0.25) (layer "B.Cu") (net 8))
 (segment (start 169.6 117.6) (end 167.2 117.6) (width 0.25) (layer "B.Cu") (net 8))
 (segment (start 167.2 117.6) (end 165.600011 116.000011) (width 0.25) (layer "B.Cu") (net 8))
 (segment (start 165.600011 116.000011) (end 161.950011 116.000011) (width 0.25) (layer "B.Cu") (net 8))
 (segment (start 166.8 120.9) (end 167.464631 120.235369) (width 0.25) (layer "F.Cu") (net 10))
 (segment (start 162.1875 123.9) (end 163.4 123.9) (width 0.25) (layer "F.Cu") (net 10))
 (segment (start 167.5375 118.657864) (end 167.464631 118.730733) (width 0.25) (layer "F.Cu") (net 10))
 (segment (start 167.464631 120.235369) (end 167.464631 118.730733) (width 0.25) (layer "F.Cu") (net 10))
 (segment (start 167.5375 117.65) (end 167.5375 118.657864) (width 0.25) (layer "F.Cu") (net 10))
 (via (at 163.4 123.9) (size 0.8) (drill 0.4) (layers "F.Cu" "B.Cu") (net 10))
 (via (at 166.8 120.9) (size 0.8) (drill 0.4) (layers "F.Cu" "B.Cu") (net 10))
 (segment (start 163.8 123.9) (end 166.8 120.9) (width 0.25) (layer "B.Cu") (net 10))
 (segment (start 163.4 123.9) (end 163.8 123.9) (width 0.25) (layer "B.Cu") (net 10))
 (segment (start 159.225 123.9) (end 160.6125 123.9) (width 0.25) (layer "F.Cu") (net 2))
 (segment (start 156.4 119.75) (end 156.4 120) (width 0.25) (layer "F.Cu") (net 6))
 (segment (start 157.681596 118.035149) (end 157.681596 118.468404) (width 0.25) (layer "F.Cu") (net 6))
 (segment (start 157.394975 117.748528) (end 157.681596 118.035149) (width 0.25) (layer "F.Cu") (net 6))
 (segment (start 157.681596 118.468404) (end 156.4 119.75) (width 0.25) (layer "F.Cu") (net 6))
 (segment (start 157.748528 117.394975) (end 158.035149 117.681596) (width 0.25) (layer "F.Cu") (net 7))
 (segment (start 163.1 119.1) (end 163.1 120) (width 0.25) (layer "F.Cu") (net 7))
 (segment (start 161.175024 117.175024) (end 163.1 119.1) (width 0.25) (layer "F.Cu") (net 7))
 (segment (start 158.035149 117.681596) (end 158.618404 117.681596) (width 0.25) (layer "F.Cu") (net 7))
 (segment (start 158.618404 117.681596) (end 159.124976 117.175024) (width 0.25) (layer "F.Cu") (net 7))
 (segment (start 159.124976 117.175024) (end 161.175024 117.175024) (width 0.25) (layer "F.Cu") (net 7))
 (segment (start 170.5 116.075) (end 169.275 116.075) (width 0.25) (layer "F.Cu") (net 11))
 (segment (start 169.275 116.075) (end 168.95 115.75) (width 0.25) (layer "F.Cu") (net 11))
 (segment (start 168.95 115.75) (end 167.5375 115.75) (width 0.25) (layer "F.Cu") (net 11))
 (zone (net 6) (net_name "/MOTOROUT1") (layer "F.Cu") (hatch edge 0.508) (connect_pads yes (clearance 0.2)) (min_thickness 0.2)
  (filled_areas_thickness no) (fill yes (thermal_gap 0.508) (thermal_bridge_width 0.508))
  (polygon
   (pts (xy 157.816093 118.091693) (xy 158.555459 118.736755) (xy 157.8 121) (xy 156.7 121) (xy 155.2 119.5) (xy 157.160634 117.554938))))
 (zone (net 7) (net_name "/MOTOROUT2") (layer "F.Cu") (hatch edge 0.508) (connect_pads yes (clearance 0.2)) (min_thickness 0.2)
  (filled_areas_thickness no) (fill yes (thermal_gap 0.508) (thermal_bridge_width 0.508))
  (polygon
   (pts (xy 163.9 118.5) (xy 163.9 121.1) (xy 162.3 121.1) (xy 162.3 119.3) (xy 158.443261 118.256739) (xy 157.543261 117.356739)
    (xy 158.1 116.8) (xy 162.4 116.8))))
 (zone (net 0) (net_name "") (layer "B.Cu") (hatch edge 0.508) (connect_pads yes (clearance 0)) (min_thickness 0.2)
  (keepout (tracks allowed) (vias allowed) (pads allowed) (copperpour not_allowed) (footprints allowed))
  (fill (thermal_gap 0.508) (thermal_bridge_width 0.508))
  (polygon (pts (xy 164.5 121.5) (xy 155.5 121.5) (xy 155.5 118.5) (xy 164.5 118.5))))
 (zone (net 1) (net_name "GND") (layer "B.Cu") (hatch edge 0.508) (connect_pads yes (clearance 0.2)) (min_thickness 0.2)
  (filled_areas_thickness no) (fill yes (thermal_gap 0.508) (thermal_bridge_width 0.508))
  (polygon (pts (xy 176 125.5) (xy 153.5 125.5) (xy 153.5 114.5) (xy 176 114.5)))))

